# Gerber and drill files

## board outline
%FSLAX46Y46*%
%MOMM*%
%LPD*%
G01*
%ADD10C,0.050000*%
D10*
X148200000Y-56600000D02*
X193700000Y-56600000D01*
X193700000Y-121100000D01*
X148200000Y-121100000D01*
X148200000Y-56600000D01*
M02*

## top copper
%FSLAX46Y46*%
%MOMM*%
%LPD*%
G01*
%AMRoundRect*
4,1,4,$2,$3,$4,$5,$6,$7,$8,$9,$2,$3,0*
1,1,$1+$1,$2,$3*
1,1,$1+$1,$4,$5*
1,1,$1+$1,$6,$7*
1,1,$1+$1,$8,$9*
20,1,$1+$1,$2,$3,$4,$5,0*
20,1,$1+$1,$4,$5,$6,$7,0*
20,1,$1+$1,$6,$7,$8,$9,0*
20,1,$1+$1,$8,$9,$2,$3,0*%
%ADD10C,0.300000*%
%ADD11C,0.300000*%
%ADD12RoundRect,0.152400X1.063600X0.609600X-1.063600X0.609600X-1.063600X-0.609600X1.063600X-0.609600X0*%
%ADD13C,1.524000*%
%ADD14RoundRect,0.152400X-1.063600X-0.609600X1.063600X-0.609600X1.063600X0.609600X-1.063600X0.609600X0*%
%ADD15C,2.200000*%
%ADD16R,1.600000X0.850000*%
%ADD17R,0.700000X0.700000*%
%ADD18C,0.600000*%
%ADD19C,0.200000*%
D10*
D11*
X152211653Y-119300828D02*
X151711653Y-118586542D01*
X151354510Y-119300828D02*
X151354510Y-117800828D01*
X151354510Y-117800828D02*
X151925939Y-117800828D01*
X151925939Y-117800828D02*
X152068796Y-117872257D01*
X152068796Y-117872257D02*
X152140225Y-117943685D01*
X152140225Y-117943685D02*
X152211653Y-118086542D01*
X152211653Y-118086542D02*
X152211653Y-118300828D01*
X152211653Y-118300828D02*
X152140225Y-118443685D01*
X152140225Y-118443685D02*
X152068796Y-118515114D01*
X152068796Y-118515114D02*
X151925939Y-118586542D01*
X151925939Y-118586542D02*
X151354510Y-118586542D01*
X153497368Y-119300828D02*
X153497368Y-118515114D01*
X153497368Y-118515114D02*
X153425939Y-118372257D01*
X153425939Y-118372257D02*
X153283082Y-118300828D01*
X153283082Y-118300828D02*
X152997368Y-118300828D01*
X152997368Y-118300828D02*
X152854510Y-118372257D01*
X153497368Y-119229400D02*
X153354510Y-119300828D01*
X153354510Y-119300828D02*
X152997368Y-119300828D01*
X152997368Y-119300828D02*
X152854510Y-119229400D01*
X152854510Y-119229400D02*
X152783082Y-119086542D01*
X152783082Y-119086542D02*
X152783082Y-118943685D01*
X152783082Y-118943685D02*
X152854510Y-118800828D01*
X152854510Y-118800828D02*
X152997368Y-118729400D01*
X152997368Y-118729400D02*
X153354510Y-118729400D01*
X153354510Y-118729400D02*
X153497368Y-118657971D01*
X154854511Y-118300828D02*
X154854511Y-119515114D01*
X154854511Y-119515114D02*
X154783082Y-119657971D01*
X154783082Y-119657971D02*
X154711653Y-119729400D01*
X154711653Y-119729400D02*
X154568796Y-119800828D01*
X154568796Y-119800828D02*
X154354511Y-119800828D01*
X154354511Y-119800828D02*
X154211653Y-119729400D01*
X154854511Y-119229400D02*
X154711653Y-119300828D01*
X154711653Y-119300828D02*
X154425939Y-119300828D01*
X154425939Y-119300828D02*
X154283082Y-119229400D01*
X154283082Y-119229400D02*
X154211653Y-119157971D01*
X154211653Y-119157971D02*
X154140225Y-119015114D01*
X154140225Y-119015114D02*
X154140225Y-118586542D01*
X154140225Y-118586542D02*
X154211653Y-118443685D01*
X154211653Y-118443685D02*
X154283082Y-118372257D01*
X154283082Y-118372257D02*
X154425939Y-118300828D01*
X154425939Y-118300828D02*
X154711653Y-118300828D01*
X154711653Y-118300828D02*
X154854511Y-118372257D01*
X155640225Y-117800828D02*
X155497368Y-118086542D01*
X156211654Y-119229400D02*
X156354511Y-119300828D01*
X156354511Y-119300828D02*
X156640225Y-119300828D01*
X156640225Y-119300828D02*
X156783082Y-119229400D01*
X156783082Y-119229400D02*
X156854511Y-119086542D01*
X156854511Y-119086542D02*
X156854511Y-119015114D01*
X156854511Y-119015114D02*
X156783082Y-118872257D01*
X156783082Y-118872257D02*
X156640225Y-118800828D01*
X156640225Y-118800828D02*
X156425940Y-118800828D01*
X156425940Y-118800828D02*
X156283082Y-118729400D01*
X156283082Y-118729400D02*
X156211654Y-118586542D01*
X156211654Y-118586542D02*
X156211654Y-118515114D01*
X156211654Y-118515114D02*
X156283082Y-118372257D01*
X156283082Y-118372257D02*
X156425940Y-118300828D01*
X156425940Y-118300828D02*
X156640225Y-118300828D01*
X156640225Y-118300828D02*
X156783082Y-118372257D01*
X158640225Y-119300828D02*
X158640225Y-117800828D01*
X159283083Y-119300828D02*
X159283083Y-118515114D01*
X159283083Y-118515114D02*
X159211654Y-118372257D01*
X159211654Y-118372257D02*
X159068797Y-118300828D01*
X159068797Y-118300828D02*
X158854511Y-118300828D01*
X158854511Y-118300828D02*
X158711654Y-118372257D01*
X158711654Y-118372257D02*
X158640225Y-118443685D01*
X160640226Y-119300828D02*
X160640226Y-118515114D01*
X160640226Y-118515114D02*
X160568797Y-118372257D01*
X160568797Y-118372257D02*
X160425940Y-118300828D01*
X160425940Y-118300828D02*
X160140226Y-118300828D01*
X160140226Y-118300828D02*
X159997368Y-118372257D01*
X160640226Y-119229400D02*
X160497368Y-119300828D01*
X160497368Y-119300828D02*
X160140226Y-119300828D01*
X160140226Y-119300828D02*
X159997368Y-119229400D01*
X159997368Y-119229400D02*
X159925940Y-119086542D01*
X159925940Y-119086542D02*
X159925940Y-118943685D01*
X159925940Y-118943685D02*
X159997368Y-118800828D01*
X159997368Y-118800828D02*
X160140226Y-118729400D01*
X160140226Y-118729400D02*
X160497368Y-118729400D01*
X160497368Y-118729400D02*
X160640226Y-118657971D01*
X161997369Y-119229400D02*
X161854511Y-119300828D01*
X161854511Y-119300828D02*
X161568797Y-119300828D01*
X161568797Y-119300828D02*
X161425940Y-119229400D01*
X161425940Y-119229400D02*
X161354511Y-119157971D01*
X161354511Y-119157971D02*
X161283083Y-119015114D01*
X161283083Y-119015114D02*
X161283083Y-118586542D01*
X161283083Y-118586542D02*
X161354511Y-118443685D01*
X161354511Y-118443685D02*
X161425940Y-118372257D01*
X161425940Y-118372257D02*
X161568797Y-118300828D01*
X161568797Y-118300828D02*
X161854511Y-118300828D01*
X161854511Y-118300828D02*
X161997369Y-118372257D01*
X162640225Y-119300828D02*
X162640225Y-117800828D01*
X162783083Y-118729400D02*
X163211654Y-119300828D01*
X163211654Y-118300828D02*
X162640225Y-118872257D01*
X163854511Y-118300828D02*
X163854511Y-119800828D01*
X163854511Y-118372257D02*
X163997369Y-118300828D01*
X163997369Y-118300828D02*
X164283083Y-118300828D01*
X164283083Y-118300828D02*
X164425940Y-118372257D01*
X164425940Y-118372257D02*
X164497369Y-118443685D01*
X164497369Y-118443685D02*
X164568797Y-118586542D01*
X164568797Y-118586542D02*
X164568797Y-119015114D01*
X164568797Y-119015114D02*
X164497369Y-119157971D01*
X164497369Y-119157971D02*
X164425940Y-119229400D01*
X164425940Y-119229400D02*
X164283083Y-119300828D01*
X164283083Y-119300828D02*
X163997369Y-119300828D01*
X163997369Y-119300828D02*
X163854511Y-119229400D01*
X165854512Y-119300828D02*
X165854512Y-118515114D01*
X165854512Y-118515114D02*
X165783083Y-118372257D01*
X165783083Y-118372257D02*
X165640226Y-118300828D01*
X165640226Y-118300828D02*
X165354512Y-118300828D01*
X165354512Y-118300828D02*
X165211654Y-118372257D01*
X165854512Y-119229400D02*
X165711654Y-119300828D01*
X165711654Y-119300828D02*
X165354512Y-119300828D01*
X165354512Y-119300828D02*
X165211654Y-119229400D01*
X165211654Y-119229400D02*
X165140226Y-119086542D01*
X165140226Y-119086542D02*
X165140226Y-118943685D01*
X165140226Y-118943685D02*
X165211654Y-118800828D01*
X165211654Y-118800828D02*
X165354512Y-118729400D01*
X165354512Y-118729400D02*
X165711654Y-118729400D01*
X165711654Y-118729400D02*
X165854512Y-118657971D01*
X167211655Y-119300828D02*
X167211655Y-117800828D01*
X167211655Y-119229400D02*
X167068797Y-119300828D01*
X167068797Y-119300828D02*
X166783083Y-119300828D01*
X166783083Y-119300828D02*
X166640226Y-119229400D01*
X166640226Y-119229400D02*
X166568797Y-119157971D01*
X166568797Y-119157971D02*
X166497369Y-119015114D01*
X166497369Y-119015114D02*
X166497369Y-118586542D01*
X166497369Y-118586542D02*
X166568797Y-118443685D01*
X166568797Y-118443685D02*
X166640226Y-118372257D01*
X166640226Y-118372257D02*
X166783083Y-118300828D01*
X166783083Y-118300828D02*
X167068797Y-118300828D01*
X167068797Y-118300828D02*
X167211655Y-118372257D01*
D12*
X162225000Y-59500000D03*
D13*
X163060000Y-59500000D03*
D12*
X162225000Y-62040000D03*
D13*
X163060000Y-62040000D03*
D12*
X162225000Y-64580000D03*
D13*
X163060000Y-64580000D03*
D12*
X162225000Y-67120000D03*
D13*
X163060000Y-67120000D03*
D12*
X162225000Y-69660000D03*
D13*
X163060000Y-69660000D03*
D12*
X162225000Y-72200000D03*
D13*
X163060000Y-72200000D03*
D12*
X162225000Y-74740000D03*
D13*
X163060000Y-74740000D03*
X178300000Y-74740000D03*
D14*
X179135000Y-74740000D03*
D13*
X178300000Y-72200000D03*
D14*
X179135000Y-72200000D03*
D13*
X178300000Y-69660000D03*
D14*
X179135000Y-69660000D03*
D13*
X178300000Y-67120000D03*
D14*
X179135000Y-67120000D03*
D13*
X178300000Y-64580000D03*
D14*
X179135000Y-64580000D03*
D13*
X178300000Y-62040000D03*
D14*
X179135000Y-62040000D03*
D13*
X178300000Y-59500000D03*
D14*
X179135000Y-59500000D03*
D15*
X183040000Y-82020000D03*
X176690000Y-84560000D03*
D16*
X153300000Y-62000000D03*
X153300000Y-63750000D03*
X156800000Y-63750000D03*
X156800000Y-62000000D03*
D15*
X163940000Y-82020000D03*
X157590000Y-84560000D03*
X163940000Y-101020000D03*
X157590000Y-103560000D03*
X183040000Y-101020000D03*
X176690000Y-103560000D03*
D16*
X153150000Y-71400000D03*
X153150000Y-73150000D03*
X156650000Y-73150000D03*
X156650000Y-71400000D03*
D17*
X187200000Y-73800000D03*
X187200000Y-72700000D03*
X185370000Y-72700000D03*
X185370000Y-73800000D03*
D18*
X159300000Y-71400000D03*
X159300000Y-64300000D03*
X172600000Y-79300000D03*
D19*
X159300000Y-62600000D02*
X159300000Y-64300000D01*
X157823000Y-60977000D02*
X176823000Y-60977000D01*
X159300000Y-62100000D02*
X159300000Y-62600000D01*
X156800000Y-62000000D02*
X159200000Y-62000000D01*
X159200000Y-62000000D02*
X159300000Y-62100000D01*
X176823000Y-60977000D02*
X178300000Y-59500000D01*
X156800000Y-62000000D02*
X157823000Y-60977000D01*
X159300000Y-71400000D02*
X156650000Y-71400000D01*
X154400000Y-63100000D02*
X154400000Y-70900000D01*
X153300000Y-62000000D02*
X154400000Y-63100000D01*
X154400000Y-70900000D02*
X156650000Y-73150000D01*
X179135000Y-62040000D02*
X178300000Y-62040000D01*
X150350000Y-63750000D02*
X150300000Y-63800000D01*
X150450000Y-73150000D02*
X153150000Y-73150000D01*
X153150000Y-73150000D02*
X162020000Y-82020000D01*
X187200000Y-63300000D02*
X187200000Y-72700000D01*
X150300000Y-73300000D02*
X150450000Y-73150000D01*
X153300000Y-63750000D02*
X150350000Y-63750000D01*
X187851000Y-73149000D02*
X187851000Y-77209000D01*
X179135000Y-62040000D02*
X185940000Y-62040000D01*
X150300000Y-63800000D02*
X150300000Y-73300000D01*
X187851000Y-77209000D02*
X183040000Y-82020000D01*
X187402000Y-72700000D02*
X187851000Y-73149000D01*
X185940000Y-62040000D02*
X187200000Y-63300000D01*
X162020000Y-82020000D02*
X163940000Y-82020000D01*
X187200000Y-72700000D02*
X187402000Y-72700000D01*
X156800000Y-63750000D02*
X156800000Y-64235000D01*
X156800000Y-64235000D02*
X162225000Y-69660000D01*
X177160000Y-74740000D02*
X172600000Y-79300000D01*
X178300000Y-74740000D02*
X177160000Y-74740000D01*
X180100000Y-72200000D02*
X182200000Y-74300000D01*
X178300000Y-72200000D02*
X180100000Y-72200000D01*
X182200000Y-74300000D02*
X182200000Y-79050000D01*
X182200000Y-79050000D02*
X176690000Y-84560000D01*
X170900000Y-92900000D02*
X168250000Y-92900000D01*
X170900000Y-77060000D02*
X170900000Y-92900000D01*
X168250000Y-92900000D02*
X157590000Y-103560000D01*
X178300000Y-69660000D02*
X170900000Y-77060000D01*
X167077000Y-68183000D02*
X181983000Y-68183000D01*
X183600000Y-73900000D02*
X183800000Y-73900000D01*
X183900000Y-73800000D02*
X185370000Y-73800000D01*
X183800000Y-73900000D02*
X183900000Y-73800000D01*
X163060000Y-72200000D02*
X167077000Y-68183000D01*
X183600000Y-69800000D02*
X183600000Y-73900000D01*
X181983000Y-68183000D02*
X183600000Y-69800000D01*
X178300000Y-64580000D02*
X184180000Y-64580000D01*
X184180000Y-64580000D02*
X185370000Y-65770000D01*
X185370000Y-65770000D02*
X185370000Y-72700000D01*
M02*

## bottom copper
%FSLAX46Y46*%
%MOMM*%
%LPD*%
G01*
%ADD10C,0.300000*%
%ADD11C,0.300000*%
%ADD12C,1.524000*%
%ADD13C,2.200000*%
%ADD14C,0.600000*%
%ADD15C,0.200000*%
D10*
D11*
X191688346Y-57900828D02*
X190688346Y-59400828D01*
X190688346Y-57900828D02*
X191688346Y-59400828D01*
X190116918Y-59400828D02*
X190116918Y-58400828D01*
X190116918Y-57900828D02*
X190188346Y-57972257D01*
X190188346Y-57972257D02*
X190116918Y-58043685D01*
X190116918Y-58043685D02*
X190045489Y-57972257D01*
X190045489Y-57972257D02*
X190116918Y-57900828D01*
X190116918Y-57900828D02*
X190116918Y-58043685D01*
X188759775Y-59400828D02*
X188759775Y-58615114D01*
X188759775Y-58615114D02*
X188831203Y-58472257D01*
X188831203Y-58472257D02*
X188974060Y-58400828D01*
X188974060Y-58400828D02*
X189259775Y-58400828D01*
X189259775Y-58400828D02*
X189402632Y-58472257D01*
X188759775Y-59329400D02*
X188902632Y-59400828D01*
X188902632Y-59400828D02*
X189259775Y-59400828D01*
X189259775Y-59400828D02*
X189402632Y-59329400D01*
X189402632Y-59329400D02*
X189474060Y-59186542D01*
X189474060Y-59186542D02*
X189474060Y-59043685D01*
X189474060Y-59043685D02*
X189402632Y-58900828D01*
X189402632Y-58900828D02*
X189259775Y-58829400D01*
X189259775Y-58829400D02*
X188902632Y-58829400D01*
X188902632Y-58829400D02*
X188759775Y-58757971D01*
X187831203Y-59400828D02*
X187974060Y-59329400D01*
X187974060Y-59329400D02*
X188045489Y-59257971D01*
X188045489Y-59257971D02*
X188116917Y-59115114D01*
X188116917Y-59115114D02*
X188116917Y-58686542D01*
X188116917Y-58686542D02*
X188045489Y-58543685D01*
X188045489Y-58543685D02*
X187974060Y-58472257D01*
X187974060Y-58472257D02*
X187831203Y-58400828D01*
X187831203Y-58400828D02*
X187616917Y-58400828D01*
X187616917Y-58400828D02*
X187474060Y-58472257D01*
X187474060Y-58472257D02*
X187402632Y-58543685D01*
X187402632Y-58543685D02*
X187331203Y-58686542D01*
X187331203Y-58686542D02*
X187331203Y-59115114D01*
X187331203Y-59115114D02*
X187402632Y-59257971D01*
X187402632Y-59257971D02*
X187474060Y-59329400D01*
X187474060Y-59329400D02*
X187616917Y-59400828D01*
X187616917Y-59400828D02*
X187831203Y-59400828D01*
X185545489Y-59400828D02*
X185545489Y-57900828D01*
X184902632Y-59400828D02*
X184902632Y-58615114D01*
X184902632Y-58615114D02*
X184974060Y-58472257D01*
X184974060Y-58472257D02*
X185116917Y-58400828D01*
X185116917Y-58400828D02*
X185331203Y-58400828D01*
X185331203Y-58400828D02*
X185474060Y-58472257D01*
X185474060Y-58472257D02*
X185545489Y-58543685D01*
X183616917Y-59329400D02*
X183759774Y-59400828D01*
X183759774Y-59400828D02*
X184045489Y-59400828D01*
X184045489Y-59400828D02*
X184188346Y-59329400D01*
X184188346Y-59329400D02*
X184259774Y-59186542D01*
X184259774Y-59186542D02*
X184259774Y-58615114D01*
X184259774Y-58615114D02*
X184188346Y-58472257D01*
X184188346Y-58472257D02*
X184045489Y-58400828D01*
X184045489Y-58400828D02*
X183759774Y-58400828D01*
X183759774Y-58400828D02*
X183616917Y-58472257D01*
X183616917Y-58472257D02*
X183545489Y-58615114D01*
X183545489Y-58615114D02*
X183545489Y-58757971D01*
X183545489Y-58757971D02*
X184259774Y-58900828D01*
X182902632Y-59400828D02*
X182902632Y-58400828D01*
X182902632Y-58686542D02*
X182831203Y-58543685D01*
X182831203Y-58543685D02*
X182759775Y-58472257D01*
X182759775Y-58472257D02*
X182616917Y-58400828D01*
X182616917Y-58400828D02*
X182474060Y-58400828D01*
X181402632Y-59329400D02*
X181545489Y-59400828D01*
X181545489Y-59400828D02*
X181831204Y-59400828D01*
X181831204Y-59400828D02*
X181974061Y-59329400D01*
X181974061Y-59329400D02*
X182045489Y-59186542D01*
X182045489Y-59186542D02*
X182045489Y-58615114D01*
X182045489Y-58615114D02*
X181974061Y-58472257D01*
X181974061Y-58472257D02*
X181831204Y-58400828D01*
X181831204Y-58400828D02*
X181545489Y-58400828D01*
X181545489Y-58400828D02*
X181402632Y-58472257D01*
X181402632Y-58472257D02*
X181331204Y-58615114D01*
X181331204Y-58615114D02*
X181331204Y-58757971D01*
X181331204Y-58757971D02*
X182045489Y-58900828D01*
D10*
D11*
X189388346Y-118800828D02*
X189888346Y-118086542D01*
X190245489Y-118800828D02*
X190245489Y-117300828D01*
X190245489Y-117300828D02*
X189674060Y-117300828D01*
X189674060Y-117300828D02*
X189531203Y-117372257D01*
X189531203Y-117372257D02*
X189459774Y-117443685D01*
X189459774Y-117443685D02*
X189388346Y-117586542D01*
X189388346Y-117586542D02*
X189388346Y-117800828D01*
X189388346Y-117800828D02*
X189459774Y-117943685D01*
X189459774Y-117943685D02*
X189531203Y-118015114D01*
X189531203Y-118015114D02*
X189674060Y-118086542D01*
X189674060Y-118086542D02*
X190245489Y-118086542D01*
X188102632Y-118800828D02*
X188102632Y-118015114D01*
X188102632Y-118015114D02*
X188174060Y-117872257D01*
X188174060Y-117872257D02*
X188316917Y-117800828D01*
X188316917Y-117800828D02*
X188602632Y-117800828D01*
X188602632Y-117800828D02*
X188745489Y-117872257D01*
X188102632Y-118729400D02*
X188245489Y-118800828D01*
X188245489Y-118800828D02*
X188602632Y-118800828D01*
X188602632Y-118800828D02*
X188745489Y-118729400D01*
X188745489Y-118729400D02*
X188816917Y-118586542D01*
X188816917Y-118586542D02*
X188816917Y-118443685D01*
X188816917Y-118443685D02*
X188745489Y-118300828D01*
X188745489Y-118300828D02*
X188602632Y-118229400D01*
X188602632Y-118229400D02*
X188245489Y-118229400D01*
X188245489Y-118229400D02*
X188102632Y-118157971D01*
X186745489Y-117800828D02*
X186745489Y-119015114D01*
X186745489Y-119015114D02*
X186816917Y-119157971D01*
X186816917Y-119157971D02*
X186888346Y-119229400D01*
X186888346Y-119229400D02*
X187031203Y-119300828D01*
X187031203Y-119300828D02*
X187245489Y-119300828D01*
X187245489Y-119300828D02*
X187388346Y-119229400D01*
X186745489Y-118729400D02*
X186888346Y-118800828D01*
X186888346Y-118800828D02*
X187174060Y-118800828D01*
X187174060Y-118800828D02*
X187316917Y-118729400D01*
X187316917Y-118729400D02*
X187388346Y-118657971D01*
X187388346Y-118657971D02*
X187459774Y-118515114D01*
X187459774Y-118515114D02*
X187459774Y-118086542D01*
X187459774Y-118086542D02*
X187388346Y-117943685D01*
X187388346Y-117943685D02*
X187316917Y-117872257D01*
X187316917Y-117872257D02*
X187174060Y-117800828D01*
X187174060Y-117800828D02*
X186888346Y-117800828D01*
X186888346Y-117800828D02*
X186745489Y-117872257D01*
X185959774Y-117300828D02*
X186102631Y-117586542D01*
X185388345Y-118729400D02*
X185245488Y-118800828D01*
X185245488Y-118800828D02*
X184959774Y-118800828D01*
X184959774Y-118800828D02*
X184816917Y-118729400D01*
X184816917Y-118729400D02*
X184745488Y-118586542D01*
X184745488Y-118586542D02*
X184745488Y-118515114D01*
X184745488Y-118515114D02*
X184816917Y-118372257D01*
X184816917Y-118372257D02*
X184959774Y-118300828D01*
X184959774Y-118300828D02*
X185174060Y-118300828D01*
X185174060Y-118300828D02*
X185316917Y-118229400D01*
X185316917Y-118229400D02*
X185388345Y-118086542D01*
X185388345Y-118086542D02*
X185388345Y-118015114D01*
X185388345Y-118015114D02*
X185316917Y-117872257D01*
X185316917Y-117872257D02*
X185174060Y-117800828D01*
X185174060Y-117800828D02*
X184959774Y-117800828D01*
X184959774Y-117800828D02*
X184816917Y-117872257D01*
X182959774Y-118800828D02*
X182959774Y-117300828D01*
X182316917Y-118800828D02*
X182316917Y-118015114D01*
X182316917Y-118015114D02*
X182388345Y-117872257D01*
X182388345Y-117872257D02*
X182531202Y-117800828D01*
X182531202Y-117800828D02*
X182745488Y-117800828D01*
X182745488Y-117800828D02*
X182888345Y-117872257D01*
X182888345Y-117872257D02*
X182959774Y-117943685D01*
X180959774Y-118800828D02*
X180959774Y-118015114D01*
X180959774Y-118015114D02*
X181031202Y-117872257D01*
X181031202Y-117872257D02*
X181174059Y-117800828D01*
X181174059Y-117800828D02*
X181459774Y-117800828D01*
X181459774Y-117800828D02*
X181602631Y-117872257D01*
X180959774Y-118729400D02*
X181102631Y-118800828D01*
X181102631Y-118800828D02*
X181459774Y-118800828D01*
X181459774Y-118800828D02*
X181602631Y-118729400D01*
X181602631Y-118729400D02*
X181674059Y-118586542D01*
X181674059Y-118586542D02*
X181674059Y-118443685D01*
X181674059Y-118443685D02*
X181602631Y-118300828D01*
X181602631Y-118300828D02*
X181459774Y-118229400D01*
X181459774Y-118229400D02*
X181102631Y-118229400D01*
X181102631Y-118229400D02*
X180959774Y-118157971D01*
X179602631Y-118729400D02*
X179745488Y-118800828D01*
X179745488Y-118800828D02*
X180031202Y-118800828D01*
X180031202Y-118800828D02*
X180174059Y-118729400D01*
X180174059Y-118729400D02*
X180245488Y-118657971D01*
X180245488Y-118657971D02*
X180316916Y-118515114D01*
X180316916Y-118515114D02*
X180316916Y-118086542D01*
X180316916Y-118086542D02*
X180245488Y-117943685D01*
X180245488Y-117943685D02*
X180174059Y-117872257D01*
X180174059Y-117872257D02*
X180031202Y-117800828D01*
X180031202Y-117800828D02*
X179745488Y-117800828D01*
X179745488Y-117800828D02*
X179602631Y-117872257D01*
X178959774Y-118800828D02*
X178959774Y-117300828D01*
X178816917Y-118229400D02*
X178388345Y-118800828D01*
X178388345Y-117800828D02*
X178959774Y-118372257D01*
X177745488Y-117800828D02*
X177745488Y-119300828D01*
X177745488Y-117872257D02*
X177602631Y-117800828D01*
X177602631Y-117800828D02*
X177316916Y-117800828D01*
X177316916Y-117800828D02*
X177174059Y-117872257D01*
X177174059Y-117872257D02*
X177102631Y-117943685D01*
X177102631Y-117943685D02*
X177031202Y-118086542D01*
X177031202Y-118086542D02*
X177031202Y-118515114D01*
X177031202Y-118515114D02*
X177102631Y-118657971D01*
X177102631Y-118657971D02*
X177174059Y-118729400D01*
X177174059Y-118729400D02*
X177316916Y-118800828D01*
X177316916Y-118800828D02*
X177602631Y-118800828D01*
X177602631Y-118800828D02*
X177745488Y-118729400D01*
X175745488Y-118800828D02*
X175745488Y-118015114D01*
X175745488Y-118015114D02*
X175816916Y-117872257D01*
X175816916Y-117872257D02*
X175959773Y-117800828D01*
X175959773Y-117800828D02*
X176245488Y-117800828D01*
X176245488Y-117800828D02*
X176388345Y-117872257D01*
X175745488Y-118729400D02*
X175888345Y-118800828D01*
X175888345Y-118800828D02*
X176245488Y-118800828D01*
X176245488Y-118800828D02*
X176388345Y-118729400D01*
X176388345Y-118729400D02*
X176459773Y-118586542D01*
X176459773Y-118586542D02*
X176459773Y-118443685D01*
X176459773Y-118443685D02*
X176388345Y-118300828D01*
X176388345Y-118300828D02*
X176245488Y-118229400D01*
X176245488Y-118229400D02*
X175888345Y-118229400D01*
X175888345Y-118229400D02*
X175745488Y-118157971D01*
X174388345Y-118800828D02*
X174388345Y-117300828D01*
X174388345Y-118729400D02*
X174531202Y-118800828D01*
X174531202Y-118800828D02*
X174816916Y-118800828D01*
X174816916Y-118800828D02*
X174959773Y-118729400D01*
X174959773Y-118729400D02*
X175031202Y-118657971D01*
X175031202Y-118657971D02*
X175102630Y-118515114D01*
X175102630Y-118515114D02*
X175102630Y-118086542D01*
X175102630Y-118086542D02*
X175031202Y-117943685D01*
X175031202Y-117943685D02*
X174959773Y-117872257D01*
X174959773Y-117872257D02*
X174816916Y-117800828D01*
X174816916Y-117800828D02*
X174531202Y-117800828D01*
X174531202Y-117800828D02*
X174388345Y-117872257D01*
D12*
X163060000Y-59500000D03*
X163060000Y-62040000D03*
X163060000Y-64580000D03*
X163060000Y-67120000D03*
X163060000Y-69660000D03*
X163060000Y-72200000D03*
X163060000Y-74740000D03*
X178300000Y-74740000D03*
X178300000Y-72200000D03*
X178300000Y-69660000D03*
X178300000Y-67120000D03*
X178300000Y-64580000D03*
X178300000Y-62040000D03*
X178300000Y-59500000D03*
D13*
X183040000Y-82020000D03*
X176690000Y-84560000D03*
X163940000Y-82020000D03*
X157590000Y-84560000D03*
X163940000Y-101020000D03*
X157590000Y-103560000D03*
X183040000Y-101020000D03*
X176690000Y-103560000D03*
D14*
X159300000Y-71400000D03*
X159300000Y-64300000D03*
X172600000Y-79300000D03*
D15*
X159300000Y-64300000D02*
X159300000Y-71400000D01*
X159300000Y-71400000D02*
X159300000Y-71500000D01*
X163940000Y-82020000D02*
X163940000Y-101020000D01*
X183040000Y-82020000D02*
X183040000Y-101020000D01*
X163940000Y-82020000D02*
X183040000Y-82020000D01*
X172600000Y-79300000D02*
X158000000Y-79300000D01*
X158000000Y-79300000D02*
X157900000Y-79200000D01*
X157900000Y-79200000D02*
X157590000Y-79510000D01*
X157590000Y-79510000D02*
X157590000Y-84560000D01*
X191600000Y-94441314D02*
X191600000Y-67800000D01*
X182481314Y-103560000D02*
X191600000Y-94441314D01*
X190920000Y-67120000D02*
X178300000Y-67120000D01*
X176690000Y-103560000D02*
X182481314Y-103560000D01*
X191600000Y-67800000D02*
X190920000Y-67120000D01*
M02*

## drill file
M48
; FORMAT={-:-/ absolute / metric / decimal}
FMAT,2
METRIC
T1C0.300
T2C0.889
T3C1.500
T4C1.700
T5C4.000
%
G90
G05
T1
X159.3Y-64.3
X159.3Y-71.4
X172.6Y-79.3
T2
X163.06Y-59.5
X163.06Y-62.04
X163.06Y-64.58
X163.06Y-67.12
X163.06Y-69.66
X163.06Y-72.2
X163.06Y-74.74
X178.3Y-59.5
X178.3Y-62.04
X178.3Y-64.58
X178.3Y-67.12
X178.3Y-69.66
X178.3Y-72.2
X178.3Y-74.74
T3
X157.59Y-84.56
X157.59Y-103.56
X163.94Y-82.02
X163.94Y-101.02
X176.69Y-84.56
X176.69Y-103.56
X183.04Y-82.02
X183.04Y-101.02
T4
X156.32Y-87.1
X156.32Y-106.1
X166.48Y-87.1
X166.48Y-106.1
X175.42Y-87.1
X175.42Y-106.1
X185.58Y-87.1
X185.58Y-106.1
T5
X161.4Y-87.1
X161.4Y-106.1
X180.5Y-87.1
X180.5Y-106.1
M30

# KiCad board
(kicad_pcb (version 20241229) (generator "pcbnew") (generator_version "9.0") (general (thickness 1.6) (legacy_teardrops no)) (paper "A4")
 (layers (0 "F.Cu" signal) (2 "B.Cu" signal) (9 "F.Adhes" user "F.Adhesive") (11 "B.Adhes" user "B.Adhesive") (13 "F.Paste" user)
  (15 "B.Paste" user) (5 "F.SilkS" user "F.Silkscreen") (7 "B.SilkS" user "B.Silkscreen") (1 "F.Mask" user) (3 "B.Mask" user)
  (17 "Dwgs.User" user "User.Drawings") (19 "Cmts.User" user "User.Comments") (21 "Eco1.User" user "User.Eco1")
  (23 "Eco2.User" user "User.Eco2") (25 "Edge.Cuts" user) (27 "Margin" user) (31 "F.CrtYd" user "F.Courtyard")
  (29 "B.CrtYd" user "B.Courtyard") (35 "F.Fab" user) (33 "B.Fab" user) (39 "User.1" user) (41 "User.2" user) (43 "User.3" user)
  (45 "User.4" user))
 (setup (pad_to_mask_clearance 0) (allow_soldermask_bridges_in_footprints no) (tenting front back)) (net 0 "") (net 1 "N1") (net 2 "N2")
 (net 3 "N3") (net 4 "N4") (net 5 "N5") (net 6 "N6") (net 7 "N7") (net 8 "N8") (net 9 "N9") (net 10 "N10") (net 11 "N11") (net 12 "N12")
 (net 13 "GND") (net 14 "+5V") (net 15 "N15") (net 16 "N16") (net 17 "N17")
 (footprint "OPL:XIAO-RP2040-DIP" (layer "F.Cu") (at 170.68 67.12)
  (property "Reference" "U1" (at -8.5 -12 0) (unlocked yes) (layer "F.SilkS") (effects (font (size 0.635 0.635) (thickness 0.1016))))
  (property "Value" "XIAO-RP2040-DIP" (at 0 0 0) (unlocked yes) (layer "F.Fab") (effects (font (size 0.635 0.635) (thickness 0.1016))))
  (pad "1" smd roundrect (at -8.455 -7.62 180) (size 2.432 1.524) (layers "F.Cu" "F.Mask") (roundrect_rratio 0.1) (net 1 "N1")
   (thermal_bridge_angle 45))
  (pad "1" thru_hole circle (at -7.62 -7.62 180) (size 1.524 1.524) (drill 0.889) (layers "*.Cu" "*.Mask") (remove_unused_layers no)
   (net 1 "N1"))
  (pad "2" smd roundrect (at -8.455 -5.08 180) (size 2.432 1.524) (layers "F.Cu" "F.Mask") (roundrect_rratio 0.1) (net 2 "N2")
   (thermal_bridge_angle 45))
  (pad "2" thru_hole circle (at -7.62 -5.08 180) (size 1.524 1.524) (drill 0.889) (layers "*.Cu" "*.Mask") (remove_unused_layers no)
   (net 2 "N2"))
  (pad "3" smd roundrect (at -8.455 -2.54 180) (size 2.432 1.524) (layers "F.Cu" "F.Mask") (roundrect_rratio 0.1) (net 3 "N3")
   (thermal_bridge_angle 45))
  (pad "3" thru_hole circle (at -7.62 -2.54 180) (size 1.524 1.524) (drill 0.889) (layers "*.Cu" "*.Mask") (remove_unused_layers no)
   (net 3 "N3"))
  (pad "4" smd roundrect (at -8.455 0 180) (size 2.432 1.524) (layers "F.Cu" "F.Mask") (roundrect_rratio 0.1) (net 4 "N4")
   (thermal_bridge_angle 45))
  (pad "4" thru_hole circle (at -7.62 0 180) (size 1.524 1.524) (drill 0.889) (layers "*.Cu" "*.Mask") (remove_unused_layers no)
   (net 4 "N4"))
  (pad "5" smd roundrect (at -8.455 2.54 180) (size 2.432 1.524) (layers "F.Cu" "F.Mask") (roundrect_rratio 0.1) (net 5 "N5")
   (thermal_bridge_angle 45))
  (pad "5" thru_hole circle (at -7.62 2.54 180) (size 1.524 1.524) (drill 0.889) (layers "*.Cu" "*.Mask") (remove_unused_layers no)
   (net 5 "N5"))
  (pad "6" smd roundrect (at -8.455 5.08 180) (size 2.432 1.524) (layers "F.Cu" "F.Mask") (roundrect_rratio 0.1) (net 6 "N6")
   (thermal_bridge_angle 45))
  (pad "6" thru_hole circle (at -7.62 5.08 180) (size 1.524 1.524) (drill 0.889) (layers "*.Cu" "*.Mask") (remove_unused_layers no)
   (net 6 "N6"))
  (pad "7" smd roundrect (at -8.455 7.62 180) (size 2.432 1.524) (layers "F.Cu" "F.Mask") (roundrect_rratio 0.1) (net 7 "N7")
   (thermal_bridge_angle 45))
  (pad "7" thru_hole circle (at -7.62 7.62 180) (size 1.524 1.524) (drill 0.889) (layers "*.Cu" "*.Mask") (remove_unused_layers no)
   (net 7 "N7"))
  (pad "8" thru_hole circle (at 7.62 7.62) (size 1.524 1.524) (drill 0.889) (layers "*.Cu" "*.Mask") (remove_unused_layers no) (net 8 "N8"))
  (pad "8" smd roundrect (at 8.455 7.62) (size 2.432 1.524) (layers "F.Cu" "F.Mask") (roundrect_rratio 0.1) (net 8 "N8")
   (thermal_bridge_angle 45))
  (pad "9" thru_hole circle (at 7.62 5.08) (size 1.524 1.524) (drill 0.889) (layers "*.Cu" "*.Mask") (remove_unused_layers no) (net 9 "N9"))
  (pad "9" smd roundrect (at 8.455 5.08) (size 2.432 1.524) (layers "F.Cu" "F.Mask") (roundrect_rratio 0.1) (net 9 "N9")
   (thermal_bridge_angle 45))
  (pad "10" thru_hole circle (at 7.62 2.54) (size 1.524 1.524) (drill 0.889) (layers "*.Cu" "*.Mask") (remove_unused_layers no)
   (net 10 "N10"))
  (pad "10" smd roundrect (at 8.455 2.54) (size 2.432 1.524) (layers "F.Cu" "F.Mask") (roundrect_rratio 0.1) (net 10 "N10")
   (thermal_bridge_angle 45))
  (pad "11" thru_hole circle (at 7.62 0) (size 1.524 1.524) (drill 0.889) (layers "*.Cu" "*.Mask") (remove_unused_layers no) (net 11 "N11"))
  (pad "11" smd roundrect (at 8.455 0) (size 2.432 1.524) (layers "F.Cu" "F.Mask") (roundrect_rratio 0.1) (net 11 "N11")
   (thermal_bridge_angle 45))
  (pad "12" thru_hole circle (at 7.62 -2.54) (size 1.524 1.524) (drill 0.889) (layers "*.Cu" "*.Mask") (remove_unused_layers no)
   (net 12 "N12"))
  (pad "12" smd roundrect (at 8.455 -2.54) (size 2.432 1.524) (layers "F.Cu" "F.Mask") (roundrect_rratio 0.1) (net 12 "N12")
   (thermal_bridge_angle 45))
  (pad "13" thru_hole circle (at 7.62 -5.08) (size 1.524 1.524) (drill 0.889) (layers "*.Cu" "*.Mask") (remove_unused_layers no)
   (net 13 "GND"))
  (pad "13" smd roundrect (at 8.455 -5.08) (size 2.432 1.524) (layers "F.Cu" "F.Mask") (roundrect_rratio 0.1) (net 13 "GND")
   (thermal_bridge_angle 45))
  (pad "14" thru_hole circle (at 7.62 -7.62) (size 1.524 1.524) (drill 0.889) (layers "*.Cu" "*.Mask") (remove_unused_layers no)
   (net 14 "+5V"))
  (pad "14" smd roundrect (at 8.455 -7.62) (size 2.432 1.524) (layers "F.Cu" "F.Mask") (roundrect_rratio 0.1) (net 14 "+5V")
   (thermal_bridge_angle 45)))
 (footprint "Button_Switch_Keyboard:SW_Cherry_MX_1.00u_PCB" (layer "F.Cu") (at 183.04 82.02)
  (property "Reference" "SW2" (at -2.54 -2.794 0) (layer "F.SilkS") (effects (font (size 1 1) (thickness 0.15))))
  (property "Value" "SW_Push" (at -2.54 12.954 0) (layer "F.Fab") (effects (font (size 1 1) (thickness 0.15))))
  (pad "" np_thru_hole circle (at -7.62 5.08) (size 1.7 1.7) (drill 1.7) (layers "*.Cu" "*.Mask"))
  (pad "" np_thru_hole circle (at -2.54 5.08) (size 4 4) (drill 4) (layers "*.Cu" "*.Mask"))
  (pad "" np_thru_hole circle (at 2.54 5.08) (size 1.7 1.7) (drill 1.7) (layers "*.Cu" "*.Mask"))
  (pad "1" thru_hole circle (at 0 0) (size 2.2 2.2) (drill 1.5) (layers "*.Cu" "*.Mask") (remove_unused_layers no) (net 13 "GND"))
  (pad "2" thru_hole circle (at -6.35 2.54) (size 2.2 2.2) (drill 1.5) (layers "*.Cu" "*.Mask") (remove_unused_layers no) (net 9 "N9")))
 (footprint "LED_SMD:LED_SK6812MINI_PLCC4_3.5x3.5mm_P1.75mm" (layer "F.Cu") (at 155.05 62.875)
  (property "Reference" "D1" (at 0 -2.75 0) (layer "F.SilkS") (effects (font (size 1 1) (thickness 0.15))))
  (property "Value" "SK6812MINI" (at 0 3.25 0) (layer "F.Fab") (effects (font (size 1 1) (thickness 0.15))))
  (pad "1" smd rect (at -1.75 -0.875) (size 1.6 0.85) (layers "F.Cu" "F.Mask" "F.Paste") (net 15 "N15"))
  (pad "2" smd rect (at -1.75 0.875) (size 1.6 0.85) (layers "F.Cu" "F.Mask" "F.Paste") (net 13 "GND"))
  (pad "3" smd rect (at 1.75 0.875) (size 1.6 0.85) (layers "F.Cu" "F.Mask" "F.Paste") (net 5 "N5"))
  (pad "4" smd rect (at 1.75 -0.875) (size 1.6 0.85) (layers "F.Cu" "F.Mask" "F.Paste") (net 14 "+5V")))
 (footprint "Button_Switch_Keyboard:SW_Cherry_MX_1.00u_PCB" (layer "F.Cu") (at 163.94 82.02)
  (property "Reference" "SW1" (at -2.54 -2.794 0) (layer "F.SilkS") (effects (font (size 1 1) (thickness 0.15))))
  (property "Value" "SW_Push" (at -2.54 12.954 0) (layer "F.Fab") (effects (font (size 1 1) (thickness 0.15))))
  (pad "" np_thru_hole circle (at -7.62 5.08) (size 1.7 1.7) (drill 1.7) (layers "*.Cu" "*.Mask"))
  (pad "" np_thru_hole circle (at -2.54 5.08) (size 4 4) (drill 4) (layers "*.Cu" "*.Mask"))
  (pad "" np_thru_hole circle (at 2.54 5.08) (size 1.7 1.7) (drill 1.7) (layers "*.Cu" "*.Mask"))
  (pad "1" thru_hole circle (at 0 0) (size 2.2 2.2) (drill 1.5) (layers "*.Cu" "*.Mask") (remove_unused_layers no) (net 13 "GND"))
  (pad "2" thru_hole circle (at -6.35 2.54) (size 2.2 2.2) (drill 1.5) (layers "*.Cu" "*.Mask") (remove_unused_layers no) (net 8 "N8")))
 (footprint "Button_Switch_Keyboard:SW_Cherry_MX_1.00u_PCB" (layer "F.Cu") (at 163.94 101.02)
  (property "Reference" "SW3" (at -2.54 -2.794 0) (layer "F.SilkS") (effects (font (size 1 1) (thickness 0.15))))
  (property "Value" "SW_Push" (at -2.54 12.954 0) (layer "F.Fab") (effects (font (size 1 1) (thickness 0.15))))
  (pad "" np_thru_hole circle (at -7.62 5.08) (size 1.7 1.7) (drill 1.7) (layers "*.Cu" "*.Mask"))
  (pad "" np_thru_hole circle (at -2.54 5.08) (size 4 4) (drill 4) (layers "*.Cu" "*.Mask"))
  (pad "" np_thru_hole circle (at 2.54 5.08) (size 1.7 1.7) (drill 1.7) (layers "*.Cu" "*.Mask"))
  (pad "1" thru_hole circle (at 0 0) (size 2.2 2.2) (drill 1.5) (layers "*.Cu" "*.Mask") (remove_unused_layers no) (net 13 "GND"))
  (pad "2" thru_hole circle (at -6.35 2.54) (size 2.2 2.2) (drill 1.5) (layers "*.Cu" "*.Mask") (remove_unused_layers no) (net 10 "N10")))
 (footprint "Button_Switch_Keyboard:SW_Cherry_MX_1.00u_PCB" (layer "F.Cu") (at 183.04 101.02)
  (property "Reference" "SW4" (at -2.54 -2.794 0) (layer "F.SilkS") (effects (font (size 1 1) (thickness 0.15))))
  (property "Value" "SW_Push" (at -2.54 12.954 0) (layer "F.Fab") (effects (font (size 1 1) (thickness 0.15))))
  (pad "" np_thru_hole circle (at -7.62 5.08) (size 1.7 1.7) (drill 1.7) (layers "*.Cu" "*.Mask"))
  (pad "" np_thru_hole circle (at -2.54 5.08) (size 4 4) (drill 4) (layers "*.Cu" "*.Mask"))
  (pad "" np_thru_hole circle (at 2.54 5.08) (size 1.7 1.7) (drill 1.7) (layers "*.Cu" "*.Mask"))
  (pad "1" thru_hole circle (at 0 0) (size 2.2 2.2) (drill 1.5) (layers "*.Cu" "*.Mask") (remove_unused_layers no) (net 13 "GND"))
  (pad "2" thru_hole circle (at -6.35 2.54) (size 2.2 2.2) (drill 1.5) (layers "*.Cu" "*.Mask") (remove_unused_layers no) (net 11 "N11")))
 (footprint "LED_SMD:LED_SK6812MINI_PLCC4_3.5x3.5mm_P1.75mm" (layer "F.Cu") (at 154.9 72.275)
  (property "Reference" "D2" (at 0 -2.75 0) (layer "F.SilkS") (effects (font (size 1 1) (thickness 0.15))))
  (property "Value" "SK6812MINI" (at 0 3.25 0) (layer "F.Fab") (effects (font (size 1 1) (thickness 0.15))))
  (pad "1" smd rect (at -1.75 -0.875) (size 1.6 0.85) (layers "F.Cu" "F.Mask" "F.Paste") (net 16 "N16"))
  (pad "2" smd rect (at -1.75 0.875) (size 1.6 0.85) (layers "F.Cu" "F.Mask" "F.Paste") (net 13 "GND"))
  (pad "3" smd rect (at 1.75 0.875) (size 1.6 0.85) (layers "F.Cu" "F.Mask" "F.Paste") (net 15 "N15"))
  (pad "4" smd rect (at 1.75 -0.875) (size 1.6 0.85) (layers "F.Cu" "F.Mask" "F.Paste") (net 14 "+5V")))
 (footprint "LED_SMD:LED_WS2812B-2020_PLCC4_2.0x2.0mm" (layer "F.Cu") (at 186.285 73.25 180)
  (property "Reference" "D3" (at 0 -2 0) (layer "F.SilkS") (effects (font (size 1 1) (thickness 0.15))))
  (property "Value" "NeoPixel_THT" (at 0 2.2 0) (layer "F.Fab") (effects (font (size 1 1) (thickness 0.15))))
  (pad "1" smd rect (at -0.915 -0.55 180) (size 0.7 0.7) (layers "F.Cu" "F.Mask" "F.Paste") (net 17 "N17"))
  (pad "2" smd rect (at -0.915 0.55 180) (size 0.7 0.7) (layers "F.Cu" "F.Mask" "F.Paste") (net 13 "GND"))
  (pad "3" smd rect (at 0.915 0.55 180) (size 0.7 0.7) (layers "F.Cu" "F.Mask" "F.Paste") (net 12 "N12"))
  (pad "4" smd rect (at 0.915 -0.55 180) (size 0.7 0.7) (layers "F.Cu" "F.Mask" "F.Paste") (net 6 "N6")))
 (gr_rect (start 148.2 56.6) (end 193.7 121.1) (stroke (width 0.05) (type default)) (fill no) (layer "Edge.Cuts"))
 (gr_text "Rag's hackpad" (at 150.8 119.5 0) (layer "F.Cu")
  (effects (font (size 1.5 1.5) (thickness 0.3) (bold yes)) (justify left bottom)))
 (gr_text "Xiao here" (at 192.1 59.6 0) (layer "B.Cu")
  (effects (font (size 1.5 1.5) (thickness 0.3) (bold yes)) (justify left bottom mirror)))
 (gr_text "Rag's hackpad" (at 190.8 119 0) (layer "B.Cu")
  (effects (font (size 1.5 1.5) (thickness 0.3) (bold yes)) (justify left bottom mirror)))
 (segment (start 159.3 62.6) (end 159.3 64.3) (width 0.2) (layer "F.Cu") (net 14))
 (segment (start 157.823 60.977) (end 176.823 60.977) (width 0.2) (layer "F.Cu") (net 14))
 (segment (start 159.3 62.1) (end 159.3 62.6) (width 0.2) (layer "F.Cu") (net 14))
 (segment (start 156.8 62) (end 159.2 62) (width 0.2) (layer "F.Cu") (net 14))
 (segment (start 159.2 62) (end 159.3 62.1) (width 0.2) (layer "F.Cu") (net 14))
 (segment (start 176.823 60.977) (end 178.3 59.5) (width 0.2) (layer "F.Cu") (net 14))
 (segment (start 156.8 62) (end 157.823 60.977) (width 0.2) (layer "F.Cu") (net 14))
 (segment (start 159.3 71.4) (end 156.65 71.4) (width 0.2) (layer "F.Cu") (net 14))
 (via (at 159.3 71.4) (size 0.6) (drill 0.3) (layers "F.Cu" "B.Cu") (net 14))
 (via (at 159.3 64.3) (size 0.6) (drill 0.3) (layers "F.Cu" "B.Cu") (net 14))
 (segment (start 159.3 64.3) (end 159.3 71.4) (width 0.2) (layer "B.Cu") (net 14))
 (segment (start 159.3 71.4) (end 159.3 71.5) (width 0.2) (layer "B.Cu") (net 14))
 (segment (start 154.4 63.1) (end 154.4 70.9) (width 0.2) (layer "F.Cu") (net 15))
 (segment (start 153.3 62) (end 154.4 63.1) (width 0.2) (layer "F.Cu") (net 15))
 (segment (start 154.4 70.9) (end 156.65 73.15) (width 0.2) (layer "F.Cu") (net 15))
 (segment (start 179.135 62.04) (end 178.3 62.04) (width 0.2) (layer "F.Cu") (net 13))
 (segment (start 150.35 63.75) (end 150.3 63.8) (width 0.2) (layer "F.Cu") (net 13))
 (segment (start 150.45 73.15) (end 153.15 73.15) (width 0.2) (layer "F.Cu") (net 13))
 (segment (start 153.15 73.15) (end 162.02 82.02) (width 0.2) (layer "F.Cu") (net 13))
 (segment (start 187.2 63.3) (end 187.2 72.7) (width 0.2) (layer "F.Cu") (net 13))
 (segment (start 150.3 73.3) (end 150.45 73.15) (width 0.2) (layer "F.Cu") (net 13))
 (segment (start 153.3 63.75) (end 150.35 63.75) (width 0.2) (layer "F.Cu") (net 13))
 (segment (start 187.851 73.149) (end 187.851 77.209) (width 0.2) (layer "F.Cu") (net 13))
 (segment (start 179.135 62.04) (end 185.94 62.04) (width 0.2) (layer "F.Cu") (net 13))
 (segment (start 150.3 63.8) (end 150.3 73.3) (width 0.2) (layer "F.Cu") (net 13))
 (segment (start 187.851 77.209) (end 183.04 82.02) (width 0.2) (layer "F.Cu") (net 13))
 (segment (start 187.402 72.7) (end 187.851 73.149) (width 0.2) (layer "F.Cu") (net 13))
 (segment (start 185.94 62.04) (end 187.2 63.3) (width 0.2) (layer "F.Cu") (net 13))
 (segment (start 162.02 82.02) (end 163.94 82.02) (width 0.2) (layer "F.Cu") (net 13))
 (segment (start 187.2 72.7) (end 187.402 72.7) (width 0.2) (layer "F.Cu") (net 13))
 (segment (start 163.94 82.02) (end 163.94 101.02) (width 0.2) (layer "B.Cu") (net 13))
 (segment (start 183.04 82.02) (end 183.04 101.02) (width 0.2) (layer "B.Cu") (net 13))
 (segment (start 163.94 82.02) (end 183.04 82.02) (width 0.2) (layer "B.Cu") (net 13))
 (segment (start 156.8 63.75) (end 156.8 64.235) (width 0.2) (layer "F.Cu") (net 5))
 (segment (start 156.8 64.235) (end 162.225 69.66) (width 0.2) (layer "F.Cu") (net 5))
 (segment (start 177.16 74.74) (end 172.6 79.3) (width 0.2) (layer "F.Cu") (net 8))
 (segment (start 178.3 74.74) (end 177.16 74.74) (width 0.2) (layer "F.Cu") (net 8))
 (via (at 172.6 79.3) (size 0.6) (drill 0.3) (layers "F.Cu" "B.Cu") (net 8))
 (segment (start 172.6 79.3) (end 158 79.3) (width 0.2) (layer "B.Cu") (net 8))
 (segment (start 158 79.3) (end 157.9 79.2) (width 0.2) (layer "B.Cu") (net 8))
 (segment (start 157.9 79.2) (end 157.59 79.51) (width 0.2) (layer "B.Cu") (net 8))
 (segment (start 157.59 79.51) (end 157.59 84.56) (width 0.2) (layer "B.Cu") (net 8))
 (segment (start 180.1 72.2) (end 182.2 74.3) (width 0.2) (layer "F.Cu") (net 9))
 (segment (start 178.3 72.2) (end 180.1 72.2) (width 0.2) (layer "F.Cu") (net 9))
 (segment (start 182.2 74.3) (end 182.2 79.05) (width 0.2) (layer "F.Cu") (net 9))
 (segment (start 182.2 79.05) (end 176.69 84.56) (width 0.2) (layer "F.Cu") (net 9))
 (segment (start 170.9 92.9) (end 168.25 92.9) (width 0.2) (layer "F.Cu") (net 10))
 (segment (start 170.9 77.06) (end 170.9 92.9) (width 0.2) (layer "F.Cu") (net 10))
 (segment (start 168.25 92.9) (end 157.59 103.56) (width 0.2) (layer "F.Cu") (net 10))
 (segment (start 178.3 69.66) (end 170.9 77.06) (width 0.2) (layer "F.Cu") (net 10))
 (segment (start 191.6 94.441314) (end 191.6 67.8) (width 0.2) (layer "B.Cu") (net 11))
 (segment (start 182.481314 103.56) (end 191.6 94.441314) (width 0.2) (layer "B.Cu") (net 11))
 (segment (start 190.92 67.12) (end 178.3 67.12) (width 0.2) (layer "B.Cu") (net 11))
 (segment (start 176.69 103.56) (end 182.481314 103.56) (width 0.2) (layer "B.Cu") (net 11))
 (segment (start 191.6 67.8) (end 190.92 67.12) (width 0.2) (layer "B.Cu") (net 11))
 (segment (start 167.077 68.183) (end 181.983 68.183) (width 0.2) (layer "F.Cu") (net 6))
 (segment (start 183.6 73.9) (end 183.8 73.9) (width 0.2) (layer "F.Cu") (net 6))
 (segment (start 183.9 73.8) (end 185.37 73.8) (width 0.2) (layer "F.Cu") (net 6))
 (segment (start 183.8 73.9) (end 183.9 73.8) (width 0.2) (layer "F.Cu") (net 6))
 (segment (start 163.06 72.2) (end 167.077 68.183) (width 0.2) (layer "F.Cu") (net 6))
 (segment (start 183.6 69.8) (end 183.6 73.9) (width 0.2) (layer "F.Cu") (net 6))
 (segment (start 181.983 68.183) (end 183.6 69.8) (width 0.2) (layer "F.Cu") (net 6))
 (segment (start 178.3 64.58) (end 184.18 64.58) (width 0.2) (layer "F.Cu") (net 12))
 (segment (start 184.18 64.58) (end 185.37 65.77) (width 0.2) (layer "F.Cu") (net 12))
 (segment (start 185.37 65.77) (end 185.37 72.7) (width 0.2) (layer "F.Cu") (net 12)))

